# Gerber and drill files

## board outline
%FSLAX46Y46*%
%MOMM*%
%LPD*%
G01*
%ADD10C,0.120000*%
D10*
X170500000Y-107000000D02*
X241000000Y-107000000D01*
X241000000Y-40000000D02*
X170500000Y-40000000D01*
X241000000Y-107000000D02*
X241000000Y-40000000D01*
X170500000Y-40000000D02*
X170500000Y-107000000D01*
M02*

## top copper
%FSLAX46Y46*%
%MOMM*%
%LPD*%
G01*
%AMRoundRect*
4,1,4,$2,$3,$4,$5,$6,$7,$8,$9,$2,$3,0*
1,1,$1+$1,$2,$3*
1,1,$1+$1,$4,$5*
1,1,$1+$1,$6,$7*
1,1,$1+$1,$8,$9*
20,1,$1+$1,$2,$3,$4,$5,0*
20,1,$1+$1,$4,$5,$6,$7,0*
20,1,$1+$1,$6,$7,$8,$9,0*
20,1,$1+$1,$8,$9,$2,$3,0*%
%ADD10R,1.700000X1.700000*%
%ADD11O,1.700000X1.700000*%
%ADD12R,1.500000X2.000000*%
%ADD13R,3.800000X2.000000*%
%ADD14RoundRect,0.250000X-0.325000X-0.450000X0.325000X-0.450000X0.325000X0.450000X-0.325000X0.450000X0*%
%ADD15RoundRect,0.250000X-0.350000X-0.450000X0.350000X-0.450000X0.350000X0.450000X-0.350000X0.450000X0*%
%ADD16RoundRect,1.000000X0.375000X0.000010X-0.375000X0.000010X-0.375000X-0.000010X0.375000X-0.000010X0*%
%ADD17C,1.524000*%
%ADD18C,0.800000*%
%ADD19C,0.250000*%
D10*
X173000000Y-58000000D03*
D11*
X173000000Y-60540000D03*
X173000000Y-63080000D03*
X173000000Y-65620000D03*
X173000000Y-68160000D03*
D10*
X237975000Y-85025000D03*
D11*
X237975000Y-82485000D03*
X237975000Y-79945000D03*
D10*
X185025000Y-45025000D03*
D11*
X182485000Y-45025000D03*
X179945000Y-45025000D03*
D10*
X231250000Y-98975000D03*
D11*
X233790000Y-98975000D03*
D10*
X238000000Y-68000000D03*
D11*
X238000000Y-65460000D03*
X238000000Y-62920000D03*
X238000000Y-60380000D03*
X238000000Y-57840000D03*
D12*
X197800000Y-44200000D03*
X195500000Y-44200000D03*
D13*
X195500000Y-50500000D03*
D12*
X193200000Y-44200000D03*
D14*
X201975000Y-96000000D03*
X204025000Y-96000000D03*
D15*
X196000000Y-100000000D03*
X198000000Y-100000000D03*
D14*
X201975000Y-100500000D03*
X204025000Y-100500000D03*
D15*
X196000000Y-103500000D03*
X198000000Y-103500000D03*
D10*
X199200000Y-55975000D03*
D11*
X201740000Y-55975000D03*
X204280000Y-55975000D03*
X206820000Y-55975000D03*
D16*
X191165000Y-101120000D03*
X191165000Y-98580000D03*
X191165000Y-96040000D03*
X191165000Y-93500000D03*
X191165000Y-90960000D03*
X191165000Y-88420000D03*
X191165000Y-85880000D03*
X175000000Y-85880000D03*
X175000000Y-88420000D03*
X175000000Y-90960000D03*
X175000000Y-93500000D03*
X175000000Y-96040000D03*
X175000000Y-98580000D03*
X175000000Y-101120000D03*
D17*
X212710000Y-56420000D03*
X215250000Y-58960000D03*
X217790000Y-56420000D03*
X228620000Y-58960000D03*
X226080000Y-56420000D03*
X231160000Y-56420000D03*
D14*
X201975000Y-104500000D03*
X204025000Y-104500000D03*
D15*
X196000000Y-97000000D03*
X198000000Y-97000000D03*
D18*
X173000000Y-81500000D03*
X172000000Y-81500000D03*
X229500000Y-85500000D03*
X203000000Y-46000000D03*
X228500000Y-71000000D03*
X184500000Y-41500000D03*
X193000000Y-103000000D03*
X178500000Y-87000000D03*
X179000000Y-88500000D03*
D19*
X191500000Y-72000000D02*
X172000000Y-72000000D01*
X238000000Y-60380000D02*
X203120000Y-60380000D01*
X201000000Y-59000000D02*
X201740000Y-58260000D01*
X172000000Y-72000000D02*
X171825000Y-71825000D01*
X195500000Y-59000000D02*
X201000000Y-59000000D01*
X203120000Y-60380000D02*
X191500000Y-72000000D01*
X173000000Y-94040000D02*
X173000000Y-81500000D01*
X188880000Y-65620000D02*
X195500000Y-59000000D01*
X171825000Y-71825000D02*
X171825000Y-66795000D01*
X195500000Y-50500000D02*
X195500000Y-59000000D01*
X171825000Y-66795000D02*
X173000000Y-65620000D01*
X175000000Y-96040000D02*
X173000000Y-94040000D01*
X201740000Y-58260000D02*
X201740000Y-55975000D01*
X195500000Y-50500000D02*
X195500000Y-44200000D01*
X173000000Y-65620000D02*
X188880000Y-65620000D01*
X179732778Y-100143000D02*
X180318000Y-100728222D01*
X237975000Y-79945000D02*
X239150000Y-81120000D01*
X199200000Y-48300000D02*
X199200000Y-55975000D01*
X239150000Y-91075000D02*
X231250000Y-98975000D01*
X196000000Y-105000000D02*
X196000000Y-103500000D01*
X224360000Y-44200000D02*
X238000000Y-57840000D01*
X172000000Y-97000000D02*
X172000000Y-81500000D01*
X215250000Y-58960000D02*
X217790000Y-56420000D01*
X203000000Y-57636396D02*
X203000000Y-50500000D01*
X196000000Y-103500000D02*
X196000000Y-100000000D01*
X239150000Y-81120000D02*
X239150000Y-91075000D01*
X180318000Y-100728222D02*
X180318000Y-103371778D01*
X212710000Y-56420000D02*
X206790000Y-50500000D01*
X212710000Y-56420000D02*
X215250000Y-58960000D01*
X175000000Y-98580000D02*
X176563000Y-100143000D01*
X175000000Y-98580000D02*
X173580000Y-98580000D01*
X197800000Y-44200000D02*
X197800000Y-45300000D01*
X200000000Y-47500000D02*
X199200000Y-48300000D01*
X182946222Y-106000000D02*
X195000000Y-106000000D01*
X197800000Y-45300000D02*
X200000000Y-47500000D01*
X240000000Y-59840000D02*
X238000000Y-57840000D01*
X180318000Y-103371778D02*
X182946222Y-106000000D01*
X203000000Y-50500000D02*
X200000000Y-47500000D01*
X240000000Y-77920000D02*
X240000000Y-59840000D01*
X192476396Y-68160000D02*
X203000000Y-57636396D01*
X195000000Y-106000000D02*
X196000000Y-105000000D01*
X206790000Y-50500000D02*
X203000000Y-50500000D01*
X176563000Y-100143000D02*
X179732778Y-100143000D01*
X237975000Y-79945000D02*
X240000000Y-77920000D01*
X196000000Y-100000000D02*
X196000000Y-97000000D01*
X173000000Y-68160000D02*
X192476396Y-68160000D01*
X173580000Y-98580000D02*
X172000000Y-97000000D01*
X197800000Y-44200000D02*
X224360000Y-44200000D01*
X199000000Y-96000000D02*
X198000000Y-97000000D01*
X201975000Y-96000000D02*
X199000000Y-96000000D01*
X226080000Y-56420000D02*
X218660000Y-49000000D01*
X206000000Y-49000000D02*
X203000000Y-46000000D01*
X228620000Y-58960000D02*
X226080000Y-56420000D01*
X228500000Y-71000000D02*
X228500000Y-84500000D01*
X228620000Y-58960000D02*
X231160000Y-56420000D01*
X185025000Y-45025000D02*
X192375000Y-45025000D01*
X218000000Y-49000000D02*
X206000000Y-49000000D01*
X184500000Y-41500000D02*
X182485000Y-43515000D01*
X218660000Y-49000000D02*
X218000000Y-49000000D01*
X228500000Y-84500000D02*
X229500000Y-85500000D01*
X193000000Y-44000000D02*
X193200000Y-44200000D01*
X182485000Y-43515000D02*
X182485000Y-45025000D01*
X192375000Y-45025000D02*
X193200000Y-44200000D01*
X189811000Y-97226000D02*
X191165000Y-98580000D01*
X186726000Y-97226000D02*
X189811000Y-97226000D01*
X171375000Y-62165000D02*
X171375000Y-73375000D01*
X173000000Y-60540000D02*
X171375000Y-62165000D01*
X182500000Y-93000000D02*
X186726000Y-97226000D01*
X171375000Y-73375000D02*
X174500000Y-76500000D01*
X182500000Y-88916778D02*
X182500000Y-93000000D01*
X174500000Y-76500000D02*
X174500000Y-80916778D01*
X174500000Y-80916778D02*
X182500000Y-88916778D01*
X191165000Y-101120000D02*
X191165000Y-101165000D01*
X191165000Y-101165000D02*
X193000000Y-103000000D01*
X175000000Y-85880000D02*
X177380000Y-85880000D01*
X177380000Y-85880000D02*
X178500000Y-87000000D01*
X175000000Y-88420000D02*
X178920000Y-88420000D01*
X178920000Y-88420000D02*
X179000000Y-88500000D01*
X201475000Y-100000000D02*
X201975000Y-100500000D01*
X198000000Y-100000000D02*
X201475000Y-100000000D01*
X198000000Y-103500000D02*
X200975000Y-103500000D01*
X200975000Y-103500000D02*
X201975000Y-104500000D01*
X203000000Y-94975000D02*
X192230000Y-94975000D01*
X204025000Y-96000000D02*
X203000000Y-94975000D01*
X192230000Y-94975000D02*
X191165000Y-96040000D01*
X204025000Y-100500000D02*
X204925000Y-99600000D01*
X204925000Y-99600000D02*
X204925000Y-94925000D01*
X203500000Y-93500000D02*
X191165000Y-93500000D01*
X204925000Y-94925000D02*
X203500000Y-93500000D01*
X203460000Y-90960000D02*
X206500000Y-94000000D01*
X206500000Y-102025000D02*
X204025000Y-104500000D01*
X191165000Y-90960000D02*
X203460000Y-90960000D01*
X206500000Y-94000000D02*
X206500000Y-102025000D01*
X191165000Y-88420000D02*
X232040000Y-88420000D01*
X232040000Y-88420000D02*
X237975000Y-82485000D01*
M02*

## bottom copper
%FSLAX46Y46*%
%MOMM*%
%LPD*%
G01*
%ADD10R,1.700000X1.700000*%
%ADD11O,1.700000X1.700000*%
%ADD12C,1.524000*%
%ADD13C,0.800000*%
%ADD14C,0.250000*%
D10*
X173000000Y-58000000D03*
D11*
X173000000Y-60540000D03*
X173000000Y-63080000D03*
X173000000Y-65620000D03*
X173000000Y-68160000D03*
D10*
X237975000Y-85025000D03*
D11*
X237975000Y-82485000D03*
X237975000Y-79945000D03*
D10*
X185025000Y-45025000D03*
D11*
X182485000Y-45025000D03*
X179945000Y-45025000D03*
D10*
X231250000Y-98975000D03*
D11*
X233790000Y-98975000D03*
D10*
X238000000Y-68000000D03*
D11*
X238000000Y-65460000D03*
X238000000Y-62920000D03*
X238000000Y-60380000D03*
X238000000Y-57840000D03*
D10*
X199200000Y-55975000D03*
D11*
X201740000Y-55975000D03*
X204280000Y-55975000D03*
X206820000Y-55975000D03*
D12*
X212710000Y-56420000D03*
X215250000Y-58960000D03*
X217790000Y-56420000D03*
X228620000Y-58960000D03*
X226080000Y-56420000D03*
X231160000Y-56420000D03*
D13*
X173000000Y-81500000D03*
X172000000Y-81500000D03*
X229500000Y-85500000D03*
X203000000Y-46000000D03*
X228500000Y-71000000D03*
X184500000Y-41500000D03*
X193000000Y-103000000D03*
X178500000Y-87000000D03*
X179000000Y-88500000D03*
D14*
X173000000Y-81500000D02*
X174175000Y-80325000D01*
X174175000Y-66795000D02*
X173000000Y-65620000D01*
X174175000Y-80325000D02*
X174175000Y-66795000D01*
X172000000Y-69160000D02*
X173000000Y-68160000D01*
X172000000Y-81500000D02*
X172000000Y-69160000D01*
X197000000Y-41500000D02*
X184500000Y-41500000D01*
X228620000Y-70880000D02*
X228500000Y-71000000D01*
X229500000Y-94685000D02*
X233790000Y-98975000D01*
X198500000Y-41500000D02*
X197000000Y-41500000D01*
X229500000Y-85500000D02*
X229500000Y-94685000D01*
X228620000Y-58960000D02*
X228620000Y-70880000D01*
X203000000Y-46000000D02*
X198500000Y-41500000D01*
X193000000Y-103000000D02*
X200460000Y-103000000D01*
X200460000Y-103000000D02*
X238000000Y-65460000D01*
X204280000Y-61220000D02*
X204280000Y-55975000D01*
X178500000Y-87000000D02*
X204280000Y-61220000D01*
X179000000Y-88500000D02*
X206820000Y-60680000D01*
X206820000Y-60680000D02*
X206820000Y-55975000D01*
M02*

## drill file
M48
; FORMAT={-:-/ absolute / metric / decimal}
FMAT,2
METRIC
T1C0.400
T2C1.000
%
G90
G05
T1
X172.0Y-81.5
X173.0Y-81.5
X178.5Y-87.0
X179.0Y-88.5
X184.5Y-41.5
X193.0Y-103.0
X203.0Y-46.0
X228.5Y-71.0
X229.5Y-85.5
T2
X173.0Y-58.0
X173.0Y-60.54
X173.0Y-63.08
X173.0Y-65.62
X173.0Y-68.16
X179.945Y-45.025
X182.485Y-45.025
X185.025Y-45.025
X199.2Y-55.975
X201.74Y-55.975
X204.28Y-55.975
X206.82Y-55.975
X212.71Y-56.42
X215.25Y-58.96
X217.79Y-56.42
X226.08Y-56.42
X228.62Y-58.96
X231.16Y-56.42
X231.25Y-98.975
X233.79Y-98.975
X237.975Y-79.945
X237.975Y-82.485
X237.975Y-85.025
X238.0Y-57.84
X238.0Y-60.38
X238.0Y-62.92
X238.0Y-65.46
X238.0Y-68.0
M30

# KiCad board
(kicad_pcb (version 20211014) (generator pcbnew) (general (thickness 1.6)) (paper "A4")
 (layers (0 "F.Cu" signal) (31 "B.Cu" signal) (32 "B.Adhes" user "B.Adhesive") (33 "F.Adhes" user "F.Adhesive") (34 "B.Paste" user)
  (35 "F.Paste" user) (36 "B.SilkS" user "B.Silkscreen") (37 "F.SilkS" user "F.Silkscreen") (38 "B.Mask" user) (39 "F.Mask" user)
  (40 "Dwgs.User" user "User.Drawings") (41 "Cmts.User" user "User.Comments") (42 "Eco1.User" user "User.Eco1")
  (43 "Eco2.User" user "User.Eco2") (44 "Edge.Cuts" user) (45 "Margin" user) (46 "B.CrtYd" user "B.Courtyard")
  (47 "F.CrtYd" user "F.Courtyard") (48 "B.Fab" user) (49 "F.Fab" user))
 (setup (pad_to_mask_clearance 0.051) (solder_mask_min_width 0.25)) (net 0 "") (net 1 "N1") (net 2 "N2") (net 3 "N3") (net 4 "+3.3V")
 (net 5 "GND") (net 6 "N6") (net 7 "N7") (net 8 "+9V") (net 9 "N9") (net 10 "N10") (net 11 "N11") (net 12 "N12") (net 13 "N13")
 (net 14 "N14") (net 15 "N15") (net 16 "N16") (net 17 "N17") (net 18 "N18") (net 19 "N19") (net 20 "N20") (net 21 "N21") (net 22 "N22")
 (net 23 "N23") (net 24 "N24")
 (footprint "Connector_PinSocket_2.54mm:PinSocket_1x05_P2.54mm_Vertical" (layer "F.Cu") (at 173 58)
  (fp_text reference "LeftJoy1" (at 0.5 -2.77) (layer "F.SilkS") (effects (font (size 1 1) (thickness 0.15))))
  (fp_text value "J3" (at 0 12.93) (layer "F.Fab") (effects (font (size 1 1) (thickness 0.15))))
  (pad "1" thru_hole rect locked (at 0 0) (size 1.7 1.7) (drill 1) (layers *.Cu *.Mask) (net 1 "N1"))
  (pad "2" thru_hole oval locked (at 0 2.54) (size 1.7 1.7) (drill 1) (layers *.Cu *.Mask) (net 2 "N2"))
  (pad "3" thru_hole oval locked (at 0 5.08) (size 1.7 1.7) (drill 1) (layers *.Cu *.Mask) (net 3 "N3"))
  (pad "4" thru_hole oval locked (at 0 7.62) (size 1.7 1.7) (drill 1) (layers *.Cu *.Mask) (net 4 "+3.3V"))
  (pad "5" thru_hole oval locked (at 0 10.16) (size 1.7 1.7) (drill 1) (layers *.Cu *.Mask) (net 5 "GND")))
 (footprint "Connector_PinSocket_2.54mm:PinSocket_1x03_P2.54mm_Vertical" (layer "F.Cu") (at 237.975 85.025 180)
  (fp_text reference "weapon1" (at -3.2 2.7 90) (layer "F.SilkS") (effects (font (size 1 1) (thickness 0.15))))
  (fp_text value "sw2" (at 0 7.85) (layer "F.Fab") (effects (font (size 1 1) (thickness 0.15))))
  (pad "1" thru_hole rect locked (at 0 0 180) (size 1.7 1.7) (drill 1) (layers *.Cu *.Mask) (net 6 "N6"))
  (pad "2" thru_hole oval locked (at 0 2.54 180) (size 1.7 1.7) (drill 1) (layers *.Cu *.Mask) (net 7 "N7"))
  (pad "3" thru_hole oval locked (at 0 5.08 180) (size 1.7 1.7) (drill 1) (layers *.Cu *.Mask) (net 5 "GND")))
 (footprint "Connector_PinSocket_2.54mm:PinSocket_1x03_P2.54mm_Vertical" (layer "F.Cu") (at 185.025 45.025 -90)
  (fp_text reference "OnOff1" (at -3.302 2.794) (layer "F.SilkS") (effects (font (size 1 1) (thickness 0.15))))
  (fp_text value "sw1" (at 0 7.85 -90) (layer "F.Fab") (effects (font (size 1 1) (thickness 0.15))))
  (pad "1" thru_hole rect locked (at 0 0 270) (size 1.7 1.7) (drill 1) (layers *.Cu *.Mask) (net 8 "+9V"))
  (pad "2" thru_hole oval locked (at 0 2.54 270) (size 1.7 1.7) (drill 1) (layers *.Cu *.Mask) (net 8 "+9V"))
  (pad "3" thru_hole oval locked (at 0 5.08 270) (size 1.7 1.7) (drill 1) (layers *.Cu *.Mask) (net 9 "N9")))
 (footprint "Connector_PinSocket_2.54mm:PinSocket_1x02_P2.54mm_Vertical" (layer "F.Cu") (at 231.25 98.975 90)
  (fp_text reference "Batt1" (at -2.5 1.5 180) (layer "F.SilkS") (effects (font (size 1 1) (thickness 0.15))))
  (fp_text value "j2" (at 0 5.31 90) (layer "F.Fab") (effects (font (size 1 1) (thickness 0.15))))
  (pad "1" thru_hole rect locked (at 0 0 90) (size 1.7 1.7) (drill 1) (layers *.Cu *.Mask) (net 5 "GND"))
  (pad "2" thru_hole oval locked (at 0 2.54 90) (size 1.7 1.7) (drill 1) (layers *.Cu *.Mask) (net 8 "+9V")))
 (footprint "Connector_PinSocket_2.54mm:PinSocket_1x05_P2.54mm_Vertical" (layer "F.Cu") (at 238 68 180)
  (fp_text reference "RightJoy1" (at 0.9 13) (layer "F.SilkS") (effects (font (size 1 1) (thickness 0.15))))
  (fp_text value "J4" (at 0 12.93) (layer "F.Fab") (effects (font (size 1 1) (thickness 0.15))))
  (pad "1" thru_hole rect locked (at 0 0 180) (size 1.7 1.7) (drill 1) (layers *.Cu *.Mask) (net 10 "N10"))
  (pad "2" thru_hole oval locked (at 0 2.54 180) (size 1.7 1.7) (drill 1) (layers *.Cu *.Mask) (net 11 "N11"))
  (pad "3" thru_hole oval locked (at 0 5.08 180) (size 1.7 1.7) (drill 1) (layers *.Cu *.Mask) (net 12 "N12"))
  (pad "4" thru_hole oval locked (at 0 7.62 180) (size 1.7 1.7) (drill 1) (layers *.Cu *.Mask) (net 4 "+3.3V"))
  (pad "5" thru_hole oval locked (at 0 10.16 180) (size 1.7 1.7) (drill 1) (layers *.Cu *.Mask) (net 5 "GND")))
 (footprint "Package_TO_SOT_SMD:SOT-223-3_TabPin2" (layer "F.Cu") (at 195.5 47.35 -90)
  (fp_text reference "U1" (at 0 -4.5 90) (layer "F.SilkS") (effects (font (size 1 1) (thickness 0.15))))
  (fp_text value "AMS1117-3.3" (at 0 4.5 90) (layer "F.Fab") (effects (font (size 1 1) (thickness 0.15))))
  (pad "1" smd rect (at -3.15 -2.3 270) (size 2 1.5) (layers "F.Cu" "F.Paste" "F.Mask") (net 5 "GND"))
  (pad "2" smd rect (at -3.15 0 270) (size 2 1.5) (layers "F.Cu" "F.Paste" "F.Mask") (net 4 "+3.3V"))
  (pad "2" smd rect (at 3.15 0 270) (size 2 3.8) (layers "F.Cu" "F.Paste" "F.Mask") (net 4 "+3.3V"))
  (pad "3" smd rect (at -3.15 2.3 270) (size 2 1.5) (layers "F.Cu" "F.Paste" "F.Mask") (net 8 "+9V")))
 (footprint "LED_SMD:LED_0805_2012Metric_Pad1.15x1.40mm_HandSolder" (layer "F.Cu") (at 203 96)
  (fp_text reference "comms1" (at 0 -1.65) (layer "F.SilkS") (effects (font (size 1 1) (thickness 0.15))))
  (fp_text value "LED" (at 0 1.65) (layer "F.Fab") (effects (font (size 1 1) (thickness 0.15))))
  (pad "1" smd roundrect (at -1.025 0) (size 1.15 1.4) (layers "F.Cu" "F.Paste" "F.Mask") (roundrect_rratio 0.217391) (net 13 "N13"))
  (pad "2" smd roundrect (at 1.025 0) (size 1.15 1.4) (layers "F.Cu" "F.Paste" "F.Mask") (roundrect_rratio 0.217391) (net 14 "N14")))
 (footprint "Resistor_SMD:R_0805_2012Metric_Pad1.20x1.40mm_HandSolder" (layer "F.Cu") (at 197 100)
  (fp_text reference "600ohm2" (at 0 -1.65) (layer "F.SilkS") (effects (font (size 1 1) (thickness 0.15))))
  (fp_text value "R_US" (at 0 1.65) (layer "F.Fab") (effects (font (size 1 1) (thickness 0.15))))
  (pad "1" smd roundrect (at -1 0) (size 1.2 1.4) (layers "F.Cu" "F.Paste" "F.Mask") (roundrect_rratio 0.208333) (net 5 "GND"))
  (pad "2" smd roundrect (at 1 0) (size 1.2 1.4) (layers "F.Cu" "F.Paste" "F.Mask") (roundrect_rratio 0.208333) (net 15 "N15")))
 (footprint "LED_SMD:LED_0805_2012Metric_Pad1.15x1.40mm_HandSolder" (layer "F.Cu") (at 203 100.5)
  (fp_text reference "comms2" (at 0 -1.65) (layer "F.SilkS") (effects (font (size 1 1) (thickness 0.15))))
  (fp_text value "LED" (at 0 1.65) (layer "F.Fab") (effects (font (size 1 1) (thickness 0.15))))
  (pad "1" smd roundrect (at -1.025 0) (size 1.15 1.4) (layers "F.Cu" "F.Paste" "F.Mask") (roundrect_rratio 0.217391) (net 15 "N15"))
  (pad "2" smd roundrect (at 1.025 0) (size 1.15 1.4) (layers "F.Cu" "F.Paste" "F.Mask") (roundrect_rratio 0.217391) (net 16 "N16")))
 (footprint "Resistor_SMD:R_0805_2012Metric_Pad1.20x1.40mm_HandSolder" (layer "F.Cu") (at 197 103.5)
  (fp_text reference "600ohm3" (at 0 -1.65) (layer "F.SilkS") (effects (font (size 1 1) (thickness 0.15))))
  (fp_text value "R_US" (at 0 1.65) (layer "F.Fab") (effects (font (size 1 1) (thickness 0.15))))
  (pad "1" smd roundrect (at -1 0) (size 1.2 1.4) (layers "F.Cu" "F.Paste" "F.Mask") (roundrect_rratio 0.208333) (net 5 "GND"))
  (pad "2" smd roundrect (at 1 0) (size 1.2 1.4) (layers "F.Cu" "F.Paste" "F.Mask") (roundrect_rratio 0.208333) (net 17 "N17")))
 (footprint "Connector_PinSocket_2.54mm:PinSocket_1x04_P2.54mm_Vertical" (layer "F.Cu") (at 199.2 55.975 90)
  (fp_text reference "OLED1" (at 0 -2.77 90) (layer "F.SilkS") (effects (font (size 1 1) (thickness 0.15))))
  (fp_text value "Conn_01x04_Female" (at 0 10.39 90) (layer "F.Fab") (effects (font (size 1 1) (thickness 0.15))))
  (pad "1" thru_hole rect (at 0 0 90) (size 1.7 1.7) (drill 1) (layers *.Cu *.Mask) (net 5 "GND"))
  (pad "2" thru_hole oval (at 0 2.54 90) (size 1.7 1.7) (drill 1) (layers *.Cu *.Mask) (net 4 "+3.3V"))
  (pad "3" thru_hole oval (at 0 5.08 90) (size 1.7 1.7) (drill 1) (layers *.Cu *.Mask) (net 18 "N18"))
  (pad "4" thru_hole oval (at 0 7.62 90) (size 1.7 1.7) (drill 1) (layers *.Cu *.Mask) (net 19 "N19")))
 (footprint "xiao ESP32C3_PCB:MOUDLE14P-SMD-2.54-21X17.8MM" (layer "F.Cu") (at 192 83 180)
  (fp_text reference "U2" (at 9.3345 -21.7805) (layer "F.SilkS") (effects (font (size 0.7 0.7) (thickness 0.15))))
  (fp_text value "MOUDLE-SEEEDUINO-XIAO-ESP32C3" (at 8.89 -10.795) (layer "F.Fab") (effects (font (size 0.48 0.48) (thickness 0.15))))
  (pad "1" smd roundrect locked (at 0.835 -18.12 180) (size 2.75 2) (layers "F.Cu" "F.Paste" "F.Mask") (roundrect_rratio 0.5) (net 11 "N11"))
  (pad "2" smd roundrect locked (at 0.835 -15.58 180) (size 2.75 2) (layers "F.Cu" "F.Paste" "F.Mask") (roundrect_rratio 0.5) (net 2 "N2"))
  (pad "3" smd roundrect locked (at 0.835 -13.04 180) (size 2.75 2) (layers "F.Cu" "F.Paste" "F.Mask") (roundrect_rratio 0.5) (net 14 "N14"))
  (pad "4" smd roundrect locked (at 0.835 -10.5 180) (size 2.75 2) (layers "F.Cu" "F.Paste" "F.Mask") (roundrect_rratio 0.5) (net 16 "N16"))
  (pad "5" smd roundrect locked (at 0.835 -7.96 180) (size 2.75 2) (layers "F.Cu" "F.Paste" "F.Mask") (roundrect_rratio 0.5) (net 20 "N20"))
  (pad "6" smd roundrect locked (at 0.835 -5.42 180) (size 2.75 2) (layers "F.Cu" "F.Paste" "F.Mask") (roundrect_rratio 0.5) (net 7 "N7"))
  (pad "7" smd roundrect locked (at 0.835 -2.88 180) (size 2.75 2) (layers "F.Cu" "F.Paste" "F.Mask") (roundrect_rratio 0.5) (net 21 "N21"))
  (pad "8" smd roundrect locked (at 17 -2.88 180) (size 2.75 2) (layers "F.Cu" "F.Paste" "F.Mask") (roundrect_rratio 0.5) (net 18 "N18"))
  (pad "9" smd roundrect locked (at 17 -5.42 180) (size 2.75 2) (layers "F.Cu" "F.Paste" "F.Mask") (roundrect_rratio 0.5) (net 19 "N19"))
  (pad "10" smd roundrect locked (at 17 -7.96 180) (size 2.75 2) (layers "F.Cu" "F.Paste" "F.Mask") (roundrect_rratio 0.5) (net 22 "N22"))
  (pad "11" smd roundrect locked (at 17 -10.5 180) (size 2.75 2) (layers "F.Cu" "F.Paste" "F.Mask") (roundrect_rratio 0.5) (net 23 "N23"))
  (pad "12" smd roundrect locked (at 17 -13.04 180) (size 2.75 2) (layers "F.Cu" "F.Paste" "F.Mask") (roundrect_rratio 0.5) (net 4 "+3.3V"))
  (pad "13" smd roundrect locked (at 17 -15.58 180) (size 2.75 2) (layers "F.Cu" "F.Paste" "F.Mask") (roundrect_rratio 0.5) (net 5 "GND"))
  (pad "14" smd roundrect locked (at 17 -18.12 180) (size 2.75 2) (layers "F.Cu" "F.Paste" "F.Mask") (roundrect_rratio 0.5) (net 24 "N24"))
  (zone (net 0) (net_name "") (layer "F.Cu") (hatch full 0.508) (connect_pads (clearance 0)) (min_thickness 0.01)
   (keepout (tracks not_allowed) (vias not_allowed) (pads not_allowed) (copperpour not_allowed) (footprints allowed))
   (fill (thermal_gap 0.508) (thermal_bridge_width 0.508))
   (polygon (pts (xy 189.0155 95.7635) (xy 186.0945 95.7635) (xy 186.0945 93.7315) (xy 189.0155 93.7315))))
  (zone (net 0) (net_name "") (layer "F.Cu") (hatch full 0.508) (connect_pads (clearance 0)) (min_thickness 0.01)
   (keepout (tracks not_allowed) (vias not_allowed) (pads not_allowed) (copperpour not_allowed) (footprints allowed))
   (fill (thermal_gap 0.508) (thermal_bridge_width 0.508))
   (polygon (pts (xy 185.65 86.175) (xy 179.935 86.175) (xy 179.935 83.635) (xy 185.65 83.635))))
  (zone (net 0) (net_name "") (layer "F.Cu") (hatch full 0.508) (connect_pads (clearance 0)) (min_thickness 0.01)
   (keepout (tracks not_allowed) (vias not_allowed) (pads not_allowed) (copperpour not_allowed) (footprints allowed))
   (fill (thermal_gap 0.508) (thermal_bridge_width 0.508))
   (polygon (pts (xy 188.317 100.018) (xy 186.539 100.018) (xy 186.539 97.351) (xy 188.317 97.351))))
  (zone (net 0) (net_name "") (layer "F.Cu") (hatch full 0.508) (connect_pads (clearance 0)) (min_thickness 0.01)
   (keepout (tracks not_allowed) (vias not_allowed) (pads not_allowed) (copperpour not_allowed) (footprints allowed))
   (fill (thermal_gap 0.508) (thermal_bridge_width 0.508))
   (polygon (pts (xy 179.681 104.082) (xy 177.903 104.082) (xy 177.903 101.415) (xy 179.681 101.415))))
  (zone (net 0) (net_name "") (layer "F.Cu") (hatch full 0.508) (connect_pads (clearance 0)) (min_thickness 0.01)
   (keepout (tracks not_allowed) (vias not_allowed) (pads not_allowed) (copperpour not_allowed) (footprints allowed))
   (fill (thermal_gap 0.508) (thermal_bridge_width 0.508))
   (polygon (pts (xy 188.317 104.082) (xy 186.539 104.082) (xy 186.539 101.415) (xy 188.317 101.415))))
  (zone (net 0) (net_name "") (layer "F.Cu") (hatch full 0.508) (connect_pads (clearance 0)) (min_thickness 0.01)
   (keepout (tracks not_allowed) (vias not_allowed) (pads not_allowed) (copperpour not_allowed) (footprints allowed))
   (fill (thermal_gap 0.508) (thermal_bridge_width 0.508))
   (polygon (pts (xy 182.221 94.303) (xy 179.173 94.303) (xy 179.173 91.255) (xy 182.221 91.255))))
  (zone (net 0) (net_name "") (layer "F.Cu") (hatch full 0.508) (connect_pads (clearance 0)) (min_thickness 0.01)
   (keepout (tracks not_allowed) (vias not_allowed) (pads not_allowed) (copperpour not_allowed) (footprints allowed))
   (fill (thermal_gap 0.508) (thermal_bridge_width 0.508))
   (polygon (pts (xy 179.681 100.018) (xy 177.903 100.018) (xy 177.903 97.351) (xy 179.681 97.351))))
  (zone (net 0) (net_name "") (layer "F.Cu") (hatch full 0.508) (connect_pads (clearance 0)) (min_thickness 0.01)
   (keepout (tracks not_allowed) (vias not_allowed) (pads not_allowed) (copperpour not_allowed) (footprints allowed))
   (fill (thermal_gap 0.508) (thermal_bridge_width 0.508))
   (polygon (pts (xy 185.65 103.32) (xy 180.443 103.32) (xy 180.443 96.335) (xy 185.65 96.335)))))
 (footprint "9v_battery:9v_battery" (layer "F.Cu") (at 221 61.5)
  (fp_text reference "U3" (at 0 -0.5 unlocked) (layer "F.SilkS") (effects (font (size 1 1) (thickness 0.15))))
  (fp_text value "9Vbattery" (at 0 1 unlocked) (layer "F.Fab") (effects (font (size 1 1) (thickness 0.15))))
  (pad "1" thru_hole circle (at -8.29 -5.08) (size 1.524 1.524) (drill 1) (layers *.Cu *.Mask) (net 5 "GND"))
  (pad "1" thru_hole circle (at -5.75 -2.54) (size 1.524 1.524) (drill 1) (layers *.Cu *.Mask) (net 5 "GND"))
  (pad "1" thru_hole circle (at -3.21 -5.08) (size 1.524 1.524) (drill 1) (layers *.Cu *.Mask) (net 5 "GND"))
  (pad "2" thru_hole circle (at 7.62 -2.54) (size 1.524 1.524) (drill 1) (layers *.Cu *.Mask) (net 8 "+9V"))
  (pad "2" thru_hole circle (at 5.08 -5.08) (size 1.524 1.524) (drill 1) (layers *.Cu *.Mask) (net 8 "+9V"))
  (pad "2" thru_hole circle (at 10.16 -5.08) (size 1.524 1.524) (drill 1) (layers *.Cu *.Mask) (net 8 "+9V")))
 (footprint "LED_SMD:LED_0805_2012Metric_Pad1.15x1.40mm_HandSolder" (layer "F.Cu") (at 203 104.5)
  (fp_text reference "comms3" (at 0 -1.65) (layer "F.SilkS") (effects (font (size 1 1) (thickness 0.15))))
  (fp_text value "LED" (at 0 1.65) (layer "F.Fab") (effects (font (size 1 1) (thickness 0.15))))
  (pad "1" smd roundrect (at -1.025 0) (size 1.15 1.4) (layers "F.Cu" "F.Paste" "F.Mask") (roundrect_rratio 0.217391) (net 17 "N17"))
  (pad "2" smd roundrect (at 1.025 0) (size 1.15 1.4) (layers "F.Cu" "F.Paste" "F.Mask") (roundrect_rratio 0.217391) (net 20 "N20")))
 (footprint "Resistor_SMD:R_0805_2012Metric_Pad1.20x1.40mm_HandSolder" (layer "F.Cu") (at 197 97)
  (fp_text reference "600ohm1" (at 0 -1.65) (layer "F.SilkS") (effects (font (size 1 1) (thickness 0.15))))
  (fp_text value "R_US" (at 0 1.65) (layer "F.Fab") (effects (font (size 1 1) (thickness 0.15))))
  (pad "1" smd roundrect (at -1 0) (size 1.2 1.4) (layers "F.Cu" "F.Paste" "F.Mask") (roundrect_rratio 0.208333) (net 5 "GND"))
  (pad "2" smd roundrect (at 1 0) (size 1.2 1.4) (layers "F.Cu" "F.Paste" "F.Mask") (roundrect_rratio 0.208333) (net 13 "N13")))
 (gr_line (start 170.5 107) (end 241 107) (layer "Edge.Cuts") (width 0.12))
 (gr_line (start 241 40) (end 170.5 40) (layer "Edge.Cuts") (width 0.12))
 (gr_line (start 241 107) (end 241 40) (layer "Edge.Cuts") (width 0.12))
 (gr_line (start 170.5 40) (end 170.5 107) (layer "Edge.Cuts") (width 0.12))
 (segment (start 191.5 72) (end 172 72) (width 0.25) (layer "F.Cu") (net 4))
 (segment (start 238 60.38) (end 203.12 60.38) (width 0.25) (layer "F.Cu") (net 4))
 (segment (start 201 59) (end 201.74 58.26) (width 0.25) (layer "F.Cu") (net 4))
 (segment (start 172 72) (end 171.825 71.825) (width 0.25) (layer "F.Cu") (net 4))
 (segment (start 195.5 59) (end 201 59) (width 0.25) (layer "F.Cu") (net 4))
 (segment (start 203.12 60.38) (end 191.5 72) (width 0.25) (layer "F.Cu") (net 4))
 (segment (start 173 94.04) (end 173 81.5) (width 0.25) (layer "F.Cu") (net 4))
 (segment (start 188.88 65.62) (end 195.5 59) (width 0.25) (layer "F.Cu") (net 4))
 (segment (start 171.825 71.825) (end 171.825 66.795) (width 0.25) (layer "F.Cu") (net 4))
 (segment (start 195.5 50.5) (end 195.5 59) (width 0.25) (layer "F.Cu") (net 4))
 (segment (start 171.825 66.795) (end 173 65.62) (width 0.25) (layer "F.Cu") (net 4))
 (segment (start 175 96.04) (end 173 94.04) (width 0.25) (layer "F.Cu") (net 4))
 (segment (start 201.74 58.26) (end 201.74 55.975) (width 0.25) (layer "F.Cu") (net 4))
 (segment (start 195.5 50.5) (end 195.5 44.2) (width 0.25) (layer "F.Cu") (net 4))
 (segment (start 173 65.62) (end 188.88 65.62) (width 0.25) (layer "F.Cu") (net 4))
 (via (at 173 81.5) (size 0.8) (drill 0.4) (layers "F.Cu" "B.Cu") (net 4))
 (segment (start 173 81.5) (end 174.175 80.325) (width 0.25) (layer "B.Cu") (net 4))
 (segment (start 174.175 66.795) (end 173 65.62) (width 0.25) (layer "B.Cu") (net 4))
 (segment (start 174.175 80.325) (end 174.175 66.795) (width 0.25) (layer "B.Cu") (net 4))
 (segment (start 179.732778 100.143) (end 180.318 100.728222) (width 0.25) (layer "F.Cu") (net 5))
 (segment (start 237.975 79.945) (end 239.15 81.12) (width 0.25) (layer "F.Cu") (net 5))
 (segment (start 199.2 48.3) (end 199.2 55.975) (width 0.25) (layer "F.Cu") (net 5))
 (segment (start 239.15 91.075) (end 231.25 98.975) (width 0.25) (layer "F.Cu") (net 5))
 (segment (start 196 105) (end 196 103.5) (width 0.25) (layer "F.Cu") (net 5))
 (segment (start 224.36 44.2) (end 238 57.84) (width 0.25) (layer "F.Cu") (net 5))
 (segment (start 172 97) (end 172 81.5) (width 0.25) (layer "F.Cu") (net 5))
 (segment (start 215.25 58.96) (end 217.79 56.42) (width 0.25) (layer "F.Cu") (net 5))
 (segment (start 203 57.636396) (end 203 50.5) (width 0.25) (layer "F.Cu") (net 5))
 (segment (start 196 103.5) (end 196 100) (width 0.25) (layer "F.Cu") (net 5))
 (segment (start 239.15 81.12) (end 239.15 91.075) (width 0.25) (layer "F.Cu") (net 5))
 (segment (start 180.318 100.728222) (end 180.318 103.371778) (width 0.25) (layer "F.Cu") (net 5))
 (segment (start 212.71 56.42) (end 206.79 50.5) (width 0.25) (layer "F.Cu") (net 5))
 (segment (start 212.71 56.42) (end 215.25 58.96) (width 0.25) (layer "F.Cu") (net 5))
 (segment (start 175 98.58) (end 176.563 100.143) (width 0.25) (layer "F.Cu") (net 5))
 (segment (start 175 98.58) (end 173.58 98.58) (width 0.25) (layer "F.Cu") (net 5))
 (segment (start 197.8 44.2) (end 197.8 45.3) (width 0.25) (layer "F.Cu") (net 5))
 (segment (start 200 47.5) (end 199.2 48.3) (width 0.25) (layer "F.Cu") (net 5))
 (segment (start 182.946222 106) (end 195 106) (width 0.25) (layer "F.Cu") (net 5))
 (segment (start 197.8 45.3) (end 200 47.5) (width 0.25) (layer "F.Cu") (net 5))
 (segment (start 240 59.84) (end 238 57.84) (width 0.25) (layer "F.Cu") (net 5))
 (segment (start 180.318 103.371778) (end 182.946222 106) (width 0.25) (layer "F.Cu") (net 5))
 (segment (start 203 50.5) (end 200 47.5) (width 0.25) (layer "F.Cu") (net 5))
 (segment (start 240 77.92) (end 240 59.84) (width 0.25) (layer "F.Cu") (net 5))
 (segment (start 192.476396 68.16) (end 203 57.636396) (width 0.25) (layer "F.Cu") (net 5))
 (segment (start 195 106) (end 196 105) (width 0.25) (layer "F.Cu") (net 5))
 (segment (start 206.79 50.5) (end 203 50.5) (width 0.25) (layer "F.Cu") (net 5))
 (segment (start 176.563 100.143) (end 179.732778 100.143) (width 0.25) (layer "F.Cu") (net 5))
 (segment (start 237.975 79.945) (end 240 77.92) (width 0.25) (layer "F.Cu") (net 5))
 (segment (start 196 100) (end 196 97) (width 0.25) (layer "F.Cu") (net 5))
 (segment (start 173 68.16) (end 192.476396 68.16) (width 0.25) (layer "F.Cu") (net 5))
 (segment (start 173.58 98.58) (end 172 97) (width 0.25) (layer "F.Cu") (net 5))
 (segment (start 197.8 44.2) (end 224.36 44.2) (width 0.25) (layer "F.Cu") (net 5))
 (via (at 172 81.5) (size 0.8) (drill 0.4) (layers "F.Cu" "B.Cu") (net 5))
 (segment (start 172 69.16) (end 173 68.16) (width 0.25) (layer "B.Cu") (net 5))
 (segment (start 172 81.5) (end 172 69.16) (width 0.25) (layer "B.Cu") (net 5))
 (segment (start 199 96) (end 198 97) (width 0.25) (layer "F.Cu") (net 13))
 (segment (start 201.975 96) (end 199 96) (width 0.25) (layer "F.Cu") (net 13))
 (segment (start 226.08 56.42) (end 218.66 49) (width 0.25) (layer "F.Cu") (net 8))
 (segment (start 206 49) (end 203 46) (width 0.25) (layer "F.Cu") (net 8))
 (segment (start 228.62 58.96) (end 226.08 56.42) (width 0.25) (layer "F.Cu") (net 8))
 (segment (start 228.5 71) (end 228.5 84.5) (width 0.25) (layer "F.Cu") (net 8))
 (segment (start 228.62 58.96) (end 231.16 56.42) (width 0.25) (layer "F.Cu") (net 8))
 (segment (start 185.025 45.025) (end 192.375 45.025) (width 0.25) (layer "F.Cu") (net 8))
 (segment (start 218 49) (end 206 49) (width 0.25) (layer "F.Cu") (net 8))
 (segment (start 184.5 41.5) (end 182.485 43.515) (width 0.25) (layer "F.Cu") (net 8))
 (segment (start 218.66 49) (end 218 49) (width 0.25) (layer "F.Cu") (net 8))
 (segment (start 228.5 84.5) (end 229.5 85.5) (width 0.25) (layer "F.Cu") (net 8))
 (segment (start 193 44) (end 193.2 44.2) (width 0.25) (layer "F.Cu") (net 8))
 (segment (start 182.485 43.515) (end 182.485 45.025) (width 0.25) (layer "F.Cu") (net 8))
 (segment (start 192.375 45.025) (end 193.2 44.2) (width 0.25) (layer "F.Cu") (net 8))
 (via (at 229.5 85.5) (size 0.8) (drill 0.4) (layers "F.Cu" "B.Cu") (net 8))
 (via (at 203 46) (size 0.8) (drill 0.4) (layers "F.Cu" "B.Cu") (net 8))
 (via (at 228.5 71) (size 0.8) (drill 0.4) (layers "F.Cu" "B.Cu") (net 8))
 (via (at 184.5 41.5) (size 0.8) (drill 0.4) (layers "F.Cu" "B.Cu") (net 8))
 (segment (start 197 41.5) (end 184.5 41.5) (width 0.25) (layer "B.Cu") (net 8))
 (segment (start 228.62 70.88) (end 228.5 71) (width 0.25) (layer "B.Cu") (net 8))
 (segment (start 229.5 94.685) (end 233.79 98.975) (width 0.25) (layer "B.Cu") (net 8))
 (segment (start 198.5 41.5) (end 197 41.5) (width 0.25) (layer "B.Cu") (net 8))
 (segment (start 229.5 85.5) (end 229.5 94.685) (width 0.25) (layer "B.Cu") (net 8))
 (segment (start 228.62 58.96) (end 228.62 70.88) (width 0.25) (layer "B.Cu") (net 8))
 (segment (start 203 46) (end 198.5 41.5) (width 0.25) (layer "B.Cu") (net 8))
 (segment (start 189.811 97.226) (end 191.165 98.58) (width 0.25) (layer "F.Cu") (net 2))
 (segment (start 186.726 97.226) (end 189.811 97.226) (width 0.25) (layer "F.Cu") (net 2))
 (segment (start 171.375 62.165) (end 171.375 73.375) (width 0.25) (layer "F.Cu") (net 2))
 (segment (start 173 60.54) (end 171.375 62.165) (width 0.25) (layer "F.Cu") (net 2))
 (segment (start 182.5 93) (end 186.726 97.226) (width 0.25) (layer "F.Cu") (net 2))
 (segment (start 171.375 73.375) (end 174.5 76.5) (width 0.25) (layer "F.Cu") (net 2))
 (segment (start 182.5 88.916778) (end 182.5 93) (width 0.25) (layer "F.Cu") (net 2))
 (segment (start 174.5 76.5) (end 174.5 80.916778) (width 0.25) (layer "F.Cu") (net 2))
 (segment (start 174.5 80.916778) (end 182.5 88.916778) (width 0.25) (layer "F.Cu") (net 2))
 (segment (start 191.165 101.12) (end 191.165 101.165) (width 0.25) (layer "F.Cu") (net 11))
 (segment (start 191.165 101.165) (end 193 103) (width 0.25) (layer "F.Cu") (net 11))
 (via (at 193 103) (size 0.8) (drill 0.4) (layers "F.Cu" "B.Cu") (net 11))
 (segment (start 193 103) (end 200.46 103) (width 0.25) (layer "B.Cu") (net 11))
 (segment (start 200.46 103) (end 238 65.46) (width 0.25) (layer "B.Cu") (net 11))
 (segment (start 175 85.88) (end 177.38 85.88) (width 0.25) (layer "F.Cu") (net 18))
 (segment (start 177.38 85.88) (end 178.5 87) (width 0.25) (layer "F.Cu") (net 18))
 (via (at 178.5 87) (size 0.8) (drill 0.4) (layers "F.Cu" "B.Cu") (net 18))
 (segment (start 204.28 61.22) (end 204.28 55.975) (width 0.25) (layer "B.Cu") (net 18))
 (segment (start 178.5 87) (end 204.28 61.22) (width 0.25) (layer "B.Cu") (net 18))
 (segment (start 175 88.42) (end 178.92 88.42) (width 0.25) (layer "F.Cu") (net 19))
 (segment (start 178.92 88.42) (end 179 88.5) (width 0.25) (layer "F.Cu") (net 19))
 (via (at 179 88.5) (size 0.8) (drill 0.4) (layers "F.Cu" "B.Cu") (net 19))
 (segment (start 179 88.5) (end 206.82 60.68) (width 0.25) (layer "B.Cu") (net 19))
 (segment (start 206.82 60.68) (end 206.82 55.975) (width 0.25) (layer "B.Cu") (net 19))
 (segment (start 201.475 100) (end 201.975 100.5) (width 0.25) (layer "F.Cu") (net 15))
 (segment (start 198 100) (end 201.475 100) (width 0.25) (layer "F.Cu") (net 15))
 (segment (start 198 103.5) (end 200.975 103.5) (width 0.25) (layer "F.Cu") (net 17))
 (segment (start 200.975 103.5) (end 201.975 104.5) (width 0.25) (layer "F.Cu") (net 17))
 (segment (start 203 94.975) (end 192.23 94.975) (width 0.25) (layer "F.Cu") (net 14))
 (segment (start 204.025 96) (end 203 94.975) (width 0.25) (layer "F.Cu") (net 14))
 (segment (start 192.23 94.975) (end 191.165 96.04) (width 0.25) (layer "F.Cu") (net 14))
 (segment (start 204.025 100.5) (end 204.925 99.6) (width 0.25) (layer "F.Cu") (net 16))
 (segment (start 204.925 99.6) (end 204.925 94.925) (width 0.25) (layer "F.Cu") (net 16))
 (segment (start 203.5 93.5) (end 191.165 93.5) (width 0.25) (layer "F.Cu") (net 16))
 (segment (start 204.925 94.925) (end 203.5 93.5) (width 0.25) (layer "F.Cu") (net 16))
 (segment (start 203.46 90.96) (end 206.5 94) (width 0.25) (layer "F.Cu") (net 20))
 (segment (start 206.5 102.025) (end 204.025 104.5) (width 0.25) (layer "F.Cu") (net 20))
 (segment (start 191.165 90.96) (end 203.46 90.96) (width 0.25) (layer "F.Cu") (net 20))
 (segment (start 206.5 94) (end 206.5 102.025) (width 0.25) (layer "F.Cu") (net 20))
 (segment (start 191.165 88.42) (end 232.04 88.42) (width 0.25) (layer "F.Cu") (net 7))
 (segment (start 232.04 88.42) (end 237.975 82.485) (width 0.25) (layer "F.Cu") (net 7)))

